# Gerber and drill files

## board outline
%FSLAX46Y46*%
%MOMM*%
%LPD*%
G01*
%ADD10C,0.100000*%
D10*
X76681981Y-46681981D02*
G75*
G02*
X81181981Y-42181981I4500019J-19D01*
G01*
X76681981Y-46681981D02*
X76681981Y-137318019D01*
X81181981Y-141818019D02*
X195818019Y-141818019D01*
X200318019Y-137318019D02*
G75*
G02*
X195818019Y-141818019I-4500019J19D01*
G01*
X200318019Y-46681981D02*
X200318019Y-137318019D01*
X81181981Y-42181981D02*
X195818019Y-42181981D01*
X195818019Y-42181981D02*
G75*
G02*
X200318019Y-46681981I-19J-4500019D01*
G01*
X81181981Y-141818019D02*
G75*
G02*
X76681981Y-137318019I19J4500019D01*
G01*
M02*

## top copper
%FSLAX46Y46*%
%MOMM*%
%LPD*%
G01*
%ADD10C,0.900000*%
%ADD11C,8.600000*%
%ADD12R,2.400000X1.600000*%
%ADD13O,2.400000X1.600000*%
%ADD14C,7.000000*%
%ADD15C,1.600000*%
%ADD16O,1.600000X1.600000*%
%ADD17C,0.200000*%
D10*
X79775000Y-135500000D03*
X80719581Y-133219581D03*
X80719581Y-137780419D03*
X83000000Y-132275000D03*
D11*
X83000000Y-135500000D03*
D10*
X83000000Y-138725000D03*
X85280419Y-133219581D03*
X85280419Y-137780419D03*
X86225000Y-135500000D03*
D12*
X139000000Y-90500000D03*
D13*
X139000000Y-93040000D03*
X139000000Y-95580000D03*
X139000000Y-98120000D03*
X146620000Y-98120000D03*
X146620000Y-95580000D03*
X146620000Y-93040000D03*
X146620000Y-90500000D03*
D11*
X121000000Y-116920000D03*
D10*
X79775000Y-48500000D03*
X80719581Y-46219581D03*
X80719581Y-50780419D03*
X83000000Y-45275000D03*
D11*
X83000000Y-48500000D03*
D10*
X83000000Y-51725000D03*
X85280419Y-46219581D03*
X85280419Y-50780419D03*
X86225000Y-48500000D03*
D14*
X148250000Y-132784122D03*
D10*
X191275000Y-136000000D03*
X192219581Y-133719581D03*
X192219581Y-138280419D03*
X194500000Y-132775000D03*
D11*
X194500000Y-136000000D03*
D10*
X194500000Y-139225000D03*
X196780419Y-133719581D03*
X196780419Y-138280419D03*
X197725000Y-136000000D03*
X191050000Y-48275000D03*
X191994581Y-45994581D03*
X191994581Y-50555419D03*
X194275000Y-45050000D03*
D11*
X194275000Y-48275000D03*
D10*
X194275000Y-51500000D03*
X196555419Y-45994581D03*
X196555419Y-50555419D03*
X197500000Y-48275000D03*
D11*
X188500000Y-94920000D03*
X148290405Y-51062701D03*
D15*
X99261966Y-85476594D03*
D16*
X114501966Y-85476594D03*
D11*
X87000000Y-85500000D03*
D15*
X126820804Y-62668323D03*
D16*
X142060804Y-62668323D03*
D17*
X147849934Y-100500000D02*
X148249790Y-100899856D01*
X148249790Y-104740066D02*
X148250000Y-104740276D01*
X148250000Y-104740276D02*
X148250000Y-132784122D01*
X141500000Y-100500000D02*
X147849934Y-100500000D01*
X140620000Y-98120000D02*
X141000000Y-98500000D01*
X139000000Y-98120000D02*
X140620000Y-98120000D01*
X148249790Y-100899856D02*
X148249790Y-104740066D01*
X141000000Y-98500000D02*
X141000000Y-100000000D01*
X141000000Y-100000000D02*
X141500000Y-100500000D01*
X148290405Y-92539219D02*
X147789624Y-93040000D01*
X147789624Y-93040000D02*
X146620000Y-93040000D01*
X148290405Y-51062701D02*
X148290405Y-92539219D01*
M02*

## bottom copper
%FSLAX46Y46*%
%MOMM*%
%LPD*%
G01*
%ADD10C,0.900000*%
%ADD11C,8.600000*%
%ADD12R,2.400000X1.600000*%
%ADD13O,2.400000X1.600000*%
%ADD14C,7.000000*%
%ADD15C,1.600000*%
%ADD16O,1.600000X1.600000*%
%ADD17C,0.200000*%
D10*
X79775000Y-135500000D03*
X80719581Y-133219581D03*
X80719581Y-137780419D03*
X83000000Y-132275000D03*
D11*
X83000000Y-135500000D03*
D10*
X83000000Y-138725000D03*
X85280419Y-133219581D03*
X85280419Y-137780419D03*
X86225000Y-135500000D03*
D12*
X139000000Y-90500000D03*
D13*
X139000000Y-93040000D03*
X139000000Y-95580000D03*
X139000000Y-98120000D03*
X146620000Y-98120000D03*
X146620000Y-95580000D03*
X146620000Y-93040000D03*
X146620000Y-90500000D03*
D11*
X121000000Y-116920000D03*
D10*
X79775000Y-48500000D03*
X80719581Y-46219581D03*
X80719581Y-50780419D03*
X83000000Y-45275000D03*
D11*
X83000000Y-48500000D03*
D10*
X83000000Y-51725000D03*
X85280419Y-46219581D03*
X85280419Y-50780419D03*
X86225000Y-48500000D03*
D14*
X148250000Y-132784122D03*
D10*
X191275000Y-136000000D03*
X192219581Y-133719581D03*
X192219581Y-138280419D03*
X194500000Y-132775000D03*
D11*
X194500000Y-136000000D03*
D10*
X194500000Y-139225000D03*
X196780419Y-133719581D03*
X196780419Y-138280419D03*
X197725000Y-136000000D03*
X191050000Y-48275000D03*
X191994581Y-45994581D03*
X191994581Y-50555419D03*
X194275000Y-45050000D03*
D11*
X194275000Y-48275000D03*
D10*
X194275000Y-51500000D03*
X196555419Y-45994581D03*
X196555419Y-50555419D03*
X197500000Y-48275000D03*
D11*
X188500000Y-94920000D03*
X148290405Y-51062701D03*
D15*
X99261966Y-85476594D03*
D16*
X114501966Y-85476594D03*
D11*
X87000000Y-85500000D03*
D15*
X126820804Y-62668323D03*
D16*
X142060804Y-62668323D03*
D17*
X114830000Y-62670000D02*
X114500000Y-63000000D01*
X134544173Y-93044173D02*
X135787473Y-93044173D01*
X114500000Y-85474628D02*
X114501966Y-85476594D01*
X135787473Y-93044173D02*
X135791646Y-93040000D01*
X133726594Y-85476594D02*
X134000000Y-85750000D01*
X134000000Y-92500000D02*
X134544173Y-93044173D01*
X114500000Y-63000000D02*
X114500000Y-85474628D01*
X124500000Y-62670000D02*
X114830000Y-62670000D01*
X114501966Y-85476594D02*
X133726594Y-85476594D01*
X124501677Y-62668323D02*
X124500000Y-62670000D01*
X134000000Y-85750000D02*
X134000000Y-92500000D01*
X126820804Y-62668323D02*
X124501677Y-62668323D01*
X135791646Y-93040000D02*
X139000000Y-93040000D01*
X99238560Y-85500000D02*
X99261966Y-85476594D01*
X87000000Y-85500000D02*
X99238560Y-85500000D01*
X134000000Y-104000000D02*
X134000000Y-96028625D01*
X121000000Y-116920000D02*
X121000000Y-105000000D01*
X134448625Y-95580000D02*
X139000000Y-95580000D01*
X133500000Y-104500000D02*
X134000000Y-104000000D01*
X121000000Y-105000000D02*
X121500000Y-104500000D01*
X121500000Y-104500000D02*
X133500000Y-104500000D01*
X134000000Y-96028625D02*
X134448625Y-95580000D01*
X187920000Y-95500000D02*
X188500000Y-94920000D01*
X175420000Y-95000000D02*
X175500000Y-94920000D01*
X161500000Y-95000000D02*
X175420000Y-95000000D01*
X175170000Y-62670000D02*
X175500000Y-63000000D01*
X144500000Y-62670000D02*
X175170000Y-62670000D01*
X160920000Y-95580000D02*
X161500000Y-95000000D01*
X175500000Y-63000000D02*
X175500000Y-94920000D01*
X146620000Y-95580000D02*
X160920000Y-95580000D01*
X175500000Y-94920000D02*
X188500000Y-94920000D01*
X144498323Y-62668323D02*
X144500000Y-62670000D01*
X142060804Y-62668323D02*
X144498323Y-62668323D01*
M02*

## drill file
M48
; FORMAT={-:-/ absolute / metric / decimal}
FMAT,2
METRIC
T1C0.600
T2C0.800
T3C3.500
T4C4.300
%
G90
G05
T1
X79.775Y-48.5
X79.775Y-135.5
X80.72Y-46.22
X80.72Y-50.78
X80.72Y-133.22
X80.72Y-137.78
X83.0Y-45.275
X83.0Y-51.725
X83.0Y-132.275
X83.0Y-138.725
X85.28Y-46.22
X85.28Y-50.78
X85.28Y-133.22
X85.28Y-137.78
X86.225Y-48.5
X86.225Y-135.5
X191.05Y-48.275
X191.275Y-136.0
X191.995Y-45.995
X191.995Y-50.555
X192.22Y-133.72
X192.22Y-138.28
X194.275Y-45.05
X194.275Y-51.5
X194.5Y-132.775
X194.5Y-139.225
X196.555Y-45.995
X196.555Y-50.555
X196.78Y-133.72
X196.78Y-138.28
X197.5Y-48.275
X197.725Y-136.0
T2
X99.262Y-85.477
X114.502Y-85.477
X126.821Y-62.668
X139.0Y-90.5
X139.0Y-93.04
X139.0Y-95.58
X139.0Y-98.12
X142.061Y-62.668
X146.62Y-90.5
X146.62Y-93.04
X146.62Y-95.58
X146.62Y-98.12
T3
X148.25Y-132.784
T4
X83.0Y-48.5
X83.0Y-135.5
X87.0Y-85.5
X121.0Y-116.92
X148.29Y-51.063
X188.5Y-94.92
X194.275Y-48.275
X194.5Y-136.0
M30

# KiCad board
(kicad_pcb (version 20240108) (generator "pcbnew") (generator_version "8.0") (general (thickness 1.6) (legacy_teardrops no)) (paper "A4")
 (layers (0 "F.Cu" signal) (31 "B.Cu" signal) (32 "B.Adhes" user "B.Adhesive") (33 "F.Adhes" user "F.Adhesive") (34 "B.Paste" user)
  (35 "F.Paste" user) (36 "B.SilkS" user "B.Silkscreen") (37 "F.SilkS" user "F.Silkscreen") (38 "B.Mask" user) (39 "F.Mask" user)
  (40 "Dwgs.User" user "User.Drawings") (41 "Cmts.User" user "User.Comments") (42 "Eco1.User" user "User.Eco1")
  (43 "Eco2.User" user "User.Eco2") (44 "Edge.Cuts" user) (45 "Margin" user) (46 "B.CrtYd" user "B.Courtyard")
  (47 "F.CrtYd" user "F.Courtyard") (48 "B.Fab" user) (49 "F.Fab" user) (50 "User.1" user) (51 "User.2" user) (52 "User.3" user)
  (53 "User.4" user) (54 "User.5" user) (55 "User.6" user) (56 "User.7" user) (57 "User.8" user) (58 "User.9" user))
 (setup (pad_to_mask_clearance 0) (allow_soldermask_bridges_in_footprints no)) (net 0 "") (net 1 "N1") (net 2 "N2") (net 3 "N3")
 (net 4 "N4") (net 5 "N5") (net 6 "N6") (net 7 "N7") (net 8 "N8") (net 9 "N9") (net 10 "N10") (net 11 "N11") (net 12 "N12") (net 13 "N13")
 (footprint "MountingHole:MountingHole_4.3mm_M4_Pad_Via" (layer "F.Cu") (at 83 135.5)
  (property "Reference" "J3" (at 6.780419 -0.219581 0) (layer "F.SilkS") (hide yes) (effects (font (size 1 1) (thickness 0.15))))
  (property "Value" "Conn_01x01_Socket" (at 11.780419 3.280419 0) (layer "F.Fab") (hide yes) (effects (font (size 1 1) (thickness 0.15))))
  (pad "1" thru_hole circle (at -3.225 0) (size 0.9 0.9) (drill 0.6) (layers "*.Cu" "*.Mask") (remove_unused_layers no) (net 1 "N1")
   (zone_connect 2))
  (pad "1" thru_hole circle (at -2.280419 -2.280419) (size 0.9 0.9) (drill 0.6) (layers "*.Cu" "*.Mask") (remove_unused_layers no)
   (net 1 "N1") (zone_connect 2))
  (pad "1" thru_hole circle (at -2.280419 2.280419) (size 0.9 0.9) (drill 0.6) (layers "*.Cu" "*.Mask") (remove_unused_layers no)
   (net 1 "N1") (zone_connect 2))
  (pad "1" thru_hole circle (at 0 -3.225) (size 0.9 0.9) (drill 0.6) (layers "*.Cu" "*.Mask") (remove_unused_layers no) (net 1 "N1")
   (zone_connect 2))
  (pad "1" thru_hole circle (at 0 0) (size 8.6 8.6) (drill 4.3) (layers "*.Cu" "*.Mask") (remove_unused_layers no) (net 1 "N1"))
  (pad "1" thru_hole circle (at 0 3.225) (size 0.9 0.9) (drill 0.6) (layers "*.Cu" "*.Mask") (remove_unused_layers no) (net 1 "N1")
   (zone_connect 2))
  (pad "1" thru_hole circle (at 2.280419 -2.280419) (size 0.9 0.9) (drill 0.6) (layers "*.Cu" "*.Mask") (remove_unused_layers no)
   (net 1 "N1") (zone_connect 2))
  (pad "1" thru_hole circle (at 2.280419 2.280419) (size 0.9 0.9) (drill 0.6) (layers "*.Cu" "*.Mask") (remove_unused_layers no)
   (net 1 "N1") (zone_connect 2))
  (pad "1" thru_hole circle (at 3.225 0) (size 0.9 0.9) (drill 0.6) (layers "*.Cu" "*.Mask") (remove_unused_layers no) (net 1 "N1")
   (zone_connect 2)))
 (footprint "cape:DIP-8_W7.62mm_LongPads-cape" (layer "F.Cu") (at 139 90.5)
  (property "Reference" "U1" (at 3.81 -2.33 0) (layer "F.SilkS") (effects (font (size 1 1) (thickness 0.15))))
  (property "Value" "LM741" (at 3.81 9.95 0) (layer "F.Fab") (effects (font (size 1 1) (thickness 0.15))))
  (pad "1" thru_hole rect (at 0 0) (size 2.4 1.6) (drill 0.8) (layers "*.Cu" "*.Mask") (remove_unused_layers no) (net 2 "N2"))
  (pad "2" thru_hole oval (at 0 2.54) (size 2.4 1.6) (drill 0.8) (layers "*.Cu" "*.Mask") (remove_unused_layers no) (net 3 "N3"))
  (pad "3" thru_hole oval (at 0 5.08) (size 2.4 1.6) (drill 0.8) (layers "*.Cu" "*.Mask") (remove_unused_layers no) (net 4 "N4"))
  (pad "4" thru_hole oval (at 0 7.62) (size 2.4 1.6) (drill 0.8) (layers "*.Cu" "*.Mask") (remove_unused_layers no) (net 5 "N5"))
  (pad "5" thru_hole oval (at 7.62 7.62) (size 2.4 1.6) (drill 0.8) (layers "*.Cu" "*.Mask") (remove_unused_layers no) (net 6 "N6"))
  (pad "6" thru_hole oval (at 7.62 5.08) (size 2.4 1.6) (drill 0.8) (layers "*.Cu" "*.Mask") (remove_unused_layers no) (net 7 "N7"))
  (pad "7" thru_hole oval (at 7.62 2.54) (size 2.4 1.6) (drill 0.8) (layers "*.Cu" "*.Mask") (remove_unused_layers no) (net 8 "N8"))
  (pad "8" thru_hole oval (at 7.62 0) (size 2.4 1.6) (drill 0.8) (layers "*.Cu" "*.Mask") (remove_unused_layers no) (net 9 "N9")))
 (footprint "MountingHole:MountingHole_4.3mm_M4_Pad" (layer "F.Cu") (at 121 116.92)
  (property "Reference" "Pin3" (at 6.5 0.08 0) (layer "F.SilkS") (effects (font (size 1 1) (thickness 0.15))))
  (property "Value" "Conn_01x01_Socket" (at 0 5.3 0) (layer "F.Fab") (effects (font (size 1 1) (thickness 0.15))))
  (pad "1" thru_hole circle (at 0 0) (size 8.6 8.6) (drill 4.3) (layers "*.Cu" "*.Mask") (remove_unused_layers no) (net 4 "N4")))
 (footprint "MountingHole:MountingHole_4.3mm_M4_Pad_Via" (layer "F.Cu") (at 83 48.5)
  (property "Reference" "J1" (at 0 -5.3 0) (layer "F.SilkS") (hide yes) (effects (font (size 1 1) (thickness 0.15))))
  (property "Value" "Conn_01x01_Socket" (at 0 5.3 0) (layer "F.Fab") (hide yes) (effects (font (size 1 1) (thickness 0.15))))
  (pad "1" thru_hole circle (at -3.225 0) (size 0.9 0.9) (drill 0.6) (layers "*.Cu" "*.Mask") (remove_unused_layers no) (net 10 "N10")
   (zone_connect 2))
  (pad "1" thru_hole circle (at -2.280419 -2.280419) (size 0.9 0.9) (drill 0.6) (layers "*.Cu" "*.Mask") (remove_unused_layers no)
   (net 10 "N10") (zone_connect 2))
  (pad "1" thru_hole circle (at -2.280419 2.280419) (size 0.9 0.9) (drill 0.6) (layers "*.Cu" "*.Mask") (remove_unused_layers no)
   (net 10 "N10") (zone_connect 2))
  (pad "1" thru_hole circle (at 0 -3.225) (size 0.9 0.9) (drill 0.6) (layers "*.Cu" "*.Mask") (remove_unused_layers no) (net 10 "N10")
   (zone_connect 2))
  (pad "1" thru_hole circle (at 0 0) (size 8.6 8.6) (drill 4.3) (layers "*.Cu" "*.Mask") (remove_unused_layers no) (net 10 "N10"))
  (pad "1" thru_hole circle (at 0 3.225) (size 0.9 0.9) (drill 0.6) (layers "*.Cu" "*.Mask") (remove_unused_layers no) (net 10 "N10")
   (zone_connect 2))
  (pad "1" thru_hole circle (at 2.280419 -2.280419) (size 0.9 0.9) (drill 0.6) (layers "*.Cu" "*.Mask") (remove_unused_layers no)
   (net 10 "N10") (zone_connect 2))
  (pad "1" thru_hole circle (at 2.280419 2.280419) (size 0.9 0.9) (drill 0.6) (layers "*.Cu" "*.Mask") (remove_unused_layers no)
   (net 10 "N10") (zone_connect 2))
  (pad "1" thru_hole circle (at 3.225 0) (size 0.9 0.9) (drill 0.6) (layers "*.Cu" "*.Mask") (remove_unused_layers no) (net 10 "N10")
   (zone_connect 2)))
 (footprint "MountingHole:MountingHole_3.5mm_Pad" (layer "F.Cu") (at 148.25 132.784122)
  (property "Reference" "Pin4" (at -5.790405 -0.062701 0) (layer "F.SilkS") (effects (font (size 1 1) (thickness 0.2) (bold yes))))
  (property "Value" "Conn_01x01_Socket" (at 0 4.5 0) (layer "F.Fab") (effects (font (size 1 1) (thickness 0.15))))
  (pad "1" thru_hole circle (at 0 0) (size 7 7) (drill 3.5) (layers "*.Cu" "*.Mask") (remove_unused_layers no) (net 5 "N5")))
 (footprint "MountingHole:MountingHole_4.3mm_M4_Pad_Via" (layer "F.Cu") (at 194.5 136)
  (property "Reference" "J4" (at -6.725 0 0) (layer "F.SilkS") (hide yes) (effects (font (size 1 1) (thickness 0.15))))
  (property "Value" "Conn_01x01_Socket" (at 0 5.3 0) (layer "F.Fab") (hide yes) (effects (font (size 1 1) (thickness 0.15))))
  (pad "1" thru_hole circle (at -3.225 0) (size 0.9 0.9) (drill 0.6) (layers "*.Cu" "*.Mask") (remove_unused_layers no) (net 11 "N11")
   (zone_connect 2))
  (pad "1" thru_hole circle (at -2.280419 -2.280419) (size 0.9 0.9) (drill 0.6) (layers "*.Cu" "*.Mask") (remove_unused_layers no)
   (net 11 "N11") (zone_connect 2))
  (pad "1" thru_hole circle (at -2.280419 2.280419) (size 0.9 0.9) (drill 0.6) (layers "*.Cu" "*.Mask") (remove_unused_layers no)
   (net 11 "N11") (zone_connect 2))
  (pad "1" thru_hole circle (at 0 -3.225) (size 0.9 0.9) (drill 0.6) (layers "*.Cu" "*.Mask") (remove_unused_layers no) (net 11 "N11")
   (zone_connect 2))
  (pad "1" thru_hole circle (at 0 0) (size 8.6 8.6) (drill 4.3) (layers "*.Cu" "*.Mask") (remove_unused_layers no) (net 11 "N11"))
  (pad "1" thru_hole circle (at 0 3.225) (size 0.9 0.9) (drill 0.6) (layers "*.Cu" "*.Mask") (remove_unused_layers no) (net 11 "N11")
   (zone_connect 2))
  (pad "1" thru_hole circle (at 2.280419 -2.280419) (size 0.9 0.9) (drill 0.6) (layers "*.Cu" "*.Mask") (remove_unused_layers no)
   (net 11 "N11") (zone_connect 2))
  (pad "1" thru_hole circle (at 2.280419 2.280419) (size 0.9 0.9) (drill 0.6) (layers "*.Cu" "*.Mask") (remove_unused_layers no)
   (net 11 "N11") (zone_connect 2))
  (pad "1" thru_hole circle (at 3.225 0) (size 0.9 0.9) (drill 0.6) (layers "*.Cu" "*.Mask") (remove_unused_layers no) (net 11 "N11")
   (zone_connect 2)))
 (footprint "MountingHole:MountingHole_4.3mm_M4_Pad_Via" (layer "F.Cu") (at 194.275 48.275)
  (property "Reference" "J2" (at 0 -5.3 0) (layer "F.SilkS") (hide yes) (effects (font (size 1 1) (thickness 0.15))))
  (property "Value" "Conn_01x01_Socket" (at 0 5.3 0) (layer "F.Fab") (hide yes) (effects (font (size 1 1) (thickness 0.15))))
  (pad "1" thru_hole circle (at -3.225 0) (size 0.9 0.9) (drill 0.6) (layers "*.Cu" "*.Mask") (remove_unused_layers no) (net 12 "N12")
   (zone_connect 2))
  (pad "1" thru_hole circle (at -2.280419 -2.280419) (size 0.9 0.9) (drill 0.6) (layers "*.Cu" "*.Mask") (remove_unused_layers no)
   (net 12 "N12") (zone_connect 2))
  (pad "1" thru_hole circle (at -2.280419 2.280419) (size 0.9 0.9) (drill 0.6) (layers "*.Cu" "*.Mask") (remove_unused_layers no)
   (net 12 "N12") (zone_connect 2))
  (pad "1" thru_hole circle (at 0 -3.225) (size 0.9 0.9) (drill 0.6) (layers "*.Cu" "*.Mask") (remove_unused_layers no) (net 12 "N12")
   (zone_connect 2))
  (pad "1" thru_hole circle (at 0 0) (size 8.6 8.6) (drill 4.3) (layers "*.Cu" "*.Mask") (remove_unused_layers no) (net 12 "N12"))
  (pad "1" thru_hole circle (at 0 3.225) (size 0.9 0.9) (drill 0.6) (layers "*.Cu" "*.Mask") (remove_unused_layers no) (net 12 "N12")
   (zone_connect 2))
  (pad "1" thru_hole circle (at 2.280419 -2.280419) (size 0.9 0.9) (drill 0.6) (layers "*.Cu" "*.Mask") (remove_unused_layers no)
   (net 12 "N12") (zone_connect 2))
  (pad "1" thru_hole circle (at 2.280419 2.280419) (size 0.9 0.9) (drill 0.6) (layers "*.Cu" "*.Mask") (remove_unused_layers no)
   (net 12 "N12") (zone_connect 2))
  (pad "1" thru_hole circle (at 3.225 0) (size 0.9 0.9) (drill 0.6) (layers "*.Cu" "*.Mask") (remove_unused_layers no) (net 12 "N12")
   (zone_connect 2)))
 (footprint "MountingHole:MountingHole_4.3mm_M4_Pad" (layer "F.Cu") (at 188.5 94.92)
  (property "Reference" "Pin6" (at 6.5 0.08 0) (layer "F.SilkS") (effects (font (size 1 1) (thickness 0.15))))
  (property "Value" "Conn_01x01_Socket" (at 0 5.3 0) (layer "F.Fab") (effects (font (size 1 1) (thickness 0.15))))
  (pad "1" thru_hole circle (at 0 0) (size 8.6 8.6) (drill 4.3) (layers "*.Cu" "*.Mask") (remove_unused_layers no) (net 7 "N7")))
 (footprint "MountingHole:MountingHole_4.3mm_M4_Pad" (layer "F.Cu") (at 148.290405 51.062701)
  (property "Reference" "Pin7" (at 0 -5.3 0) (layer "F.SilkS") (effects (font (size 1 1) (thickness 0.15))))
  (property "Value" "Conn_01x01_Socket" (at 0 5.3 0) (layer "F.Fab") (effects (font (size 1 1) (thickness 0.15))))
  (pad "1" thru_hole circle (at 0 0) (size 8.6 8.6) (drill 4.3) (layers "*.Cu" "*.Mask") (remove_unused_layers no) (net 8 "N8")))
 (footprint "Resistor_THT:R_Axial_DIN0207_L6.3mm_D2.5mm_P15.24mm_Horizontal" (layer "F.Cu") (at 99.261966 85.476594)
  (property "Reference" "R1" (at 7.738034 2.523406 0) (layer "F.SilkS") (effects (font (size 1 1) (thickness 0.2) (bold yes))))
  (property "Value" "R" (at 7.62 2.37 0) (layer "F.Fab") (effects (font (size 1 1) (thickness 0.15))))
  (pad "1" thru_hole circle (at 0 0) (size 1.6 1.6) (drill 0.8) (layers "*.Cu" "*.Mask") (remove_unused_layers no) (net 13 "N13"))
  (pad "2" thru_hole oval (at 15.24 0) (size 1.6 1.6) (drill 0.8) (layers "*.Cu" "*.Mask") (remove_unused_layers no) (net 3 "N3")))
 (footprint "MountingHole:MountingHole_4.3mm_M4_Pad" (layer "F.Cu") (at 87 85.5)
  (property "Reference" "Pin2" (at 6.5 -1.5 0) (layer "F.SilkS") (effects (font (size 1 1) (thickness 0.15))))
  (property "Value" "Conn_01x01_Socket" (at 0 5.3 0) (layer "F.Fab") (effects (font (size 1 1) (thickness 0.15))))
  (pad "1" thru_hole circle (at 0 0) (size 8.6 8.6) (drill 4.3) (layers "*.Cu" "*.Mask") (remove_unused_layers no) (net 13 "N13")))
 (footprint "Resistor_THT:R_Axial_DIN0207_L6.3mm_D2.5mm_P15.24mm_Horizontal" (layer "F.Cu") (at 126.820804 62.668323)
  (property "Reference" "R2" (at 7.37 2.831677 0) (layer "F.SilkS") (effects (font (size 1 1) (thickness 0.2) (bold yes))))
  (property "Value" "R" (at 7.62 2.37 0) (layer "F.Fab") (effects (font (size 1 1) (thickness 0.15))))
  (pad "1" thru_hole circle (at 0 0) (size 1.6 1.6) (drill 0.8) (layers "*.Cu" "*.Mask") (remove_unused_layers no) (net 3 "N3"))
  (pad "2" thru_hole oval (at 15.24 0) (size 1.6 1.6) (drill 0.8) (layers "*.Cu" "*.Mask") (remove_unused_layers no) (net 7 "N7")))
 (gr_arc (start 76.681981 46.681981) (mid 78 43.5) (end 81.181981 42.181981) (stroke (width 0.1) (type default)) (layer "Edge.Cuts"))
 (gr_line (start 76.681981 46.681981) (end 76.681981 137.318019) (stroke (width 0.1) (type default)) (layer "Edge.Cuts"))
 (gr_line (start 81.181981 141.818019) (end 195.818019 141.818019) (stroke (width 0.1) (type default)) (layer "Edge.Cuts"))
 (gr_arc (start 200.318019 137.318019) (mid 199 140.5) (end 195.818019 141.818019) (stroke (width 0.1) (type default)) (layer "Edge.Cuts"))
 (gr_line (start 200.318019 46.681981) (end 200.318019 137.318019) (stroke (width 0.1) (type default)) (layer "Edge.Cuts"))
 (gr_line (start 81.181981 42.181981) (end 195.818019 42.181981) (stroke (width 0.1) (type default)) (layer "Edge.Cuts"))
 (gr_arc (start 195.818019 42.181981) (mid 199 43.5) (end 200.318019 46.681981) (stroke (width 0.1) (type default)) (layer "Edge.Cuts"))
 (gr_arc (start 81.181981 141.818019) (mid 78 140.5) (end 76.681981 137.318019) (stroke (width 0.1) (type default)) (layer "Edge.Cuts"))
 (segment (start 114.83 62.67) (end 114.5 63) (width 0.2) (layer "B.Cu") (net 3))
 (segment (start 134.544173 93.044173) (end 135.787473 93.044173) (width 0.2) (layer "B.Cu") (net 3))
 (segment (start 114.5 85.474628) (end 114.501966 85.476594) (width 0.2) (layer "B.Cu") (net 3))
 (segment (start 135.787473 93.044173) (end 135.791646 93.04) (width 0.2) (layer "B.Cu") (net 3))
 (segment (start 133.726594 85.476594) (end 134 85.75) (width 0.2) (layer "B.Cu") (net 3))
 (segment (start 134 92.5) (end 134.544173 93.044173) (width 0.2) (layer "B.Cu") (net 3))
 (segment (start 114.5 63) (end 114.5 85.474628) (width 0.2) (layer "B.Cu") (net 3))
 (segment (start 124.5 62.67) (end 114.83 62.67) (width 0.2) (layer "B.Cu") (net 3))
 (segment (start 114.501966 85.476594) (end 133.726594 85.476594) (width 0.2) (layer "B.Cu") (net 3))
 (segment (start 124.501677 62.668323) (end 124.5 62.67) (width 0.2) (layer "B.Cu") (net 3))
 (segment (start 134 85.75) (end 134 92.5) (width 0.2) (layer "B.Cu") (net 3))
 (segment (start 126.820804 62.668323) (end 124.501677 62.668323) (width 0.2) (layer "B.Cu") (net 3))
 (segment (start 135.791646 93.04) (end 139 93.04) (width 0.2) (layer "B.Cu") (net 3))
 (segment (start 99.23856 85.5) (end 99.261966 85.476594) (width 0.2) (layer "B.Cu") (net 13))
 (segment (start 87 85.5) (end 99.23856 85.5) (width 0.2) (layer "B.Cu") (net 13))
 (segment (start 134 104) (end 134 96.028625) (width 0.2) (layer "B.Cu") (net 4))
 (segment (start 121 116.92) (end 121 105) (width 0.2) (layer "B.Cu") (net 4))
 (segment (start 134.448625 95.58) (end 139 95.58) (width 0.2) (layer "B.Cu") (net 4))
 (segment (start 133.5 104.5) (end 134 104) (width 0.2) (layer "B.Cu") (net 4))
 (segment (start 121 105) (end 121.5 104.5) (width 0.2) (layer "B.Cu") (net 4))
 (segment (start 121.5 104.5) (end 133.5 104.5) (width 0.2) (layer "B.Cu") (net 4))
 (segment (start 134 96.028625) (end 134.448625 95.58) (width 0.2) (layer "B.Cu") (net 4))
 (segment (start 147.849934 100.5) (end 148.24979 100.899856) (width 0.2) (layer "F.Cu") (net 5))
 (segment (start 148.24979 104.740066) (end 148.25 104.740276) (width 0.2) (layer "F.Cu") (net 5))
 (segment (start 148.25 104.740276) (end 148.25 132.784122) (width 0.2) (layer "F.Cu") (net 5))
 (segment (start 141.5 100.5) (end 147.849934 100.5) (width 0.2) (layer "F.Cu") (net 5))
 (segment (start 140.62 98.12) (end 141 98.5) (width 0.2) (layer "F.Cu") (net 5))
 (segment (start 139 98.12) (end 140.62 98.12) (width 0.2) (layer "F.Cu") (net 5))
 (segment (start 148.24979 100.899856) (end 148.24979 104.740066) (width 0.2) (layer "F.Cu") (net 5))
 (segment (start 141 98.5) (end 141 100) (width 0.2) (layer "F.Cu") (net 5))
 (segment (start 141 100) (end 141.5 100.5) (width 0.2) (layer "F.Cu") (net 5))
 (segment (start 187.92 95.5) (end 188.5 94.92) (width 0.2) (layer "B.Cu") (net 7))
 (segment (start 175.42 95) (end 175.5 94.92) (width 0.2) (layer "B.Cu") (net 7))
 (segment (start 161.5 95) (end 175.42 95) (width 0.2) (layer "B.Cu") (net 7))
 (segment (start 175.17 62.67) (end 175.5 63) (width 0.2) (layer "B.Cu") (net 7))
 (segment (start 144.5 62.67) (end 175.17 62.67) (width 0.2) (layer "B.Cu") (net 7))
 (segment (start 160.92 95.58) (end 161.5 95) (width 0.2) (layer "B.Cu") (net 7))
 (segment (start 175.5 63) (end 175.5 94.92) (width 0.2) (layer "B.Cu") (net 7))
 (segment (start 146.62 95.58) (end 160.92 95.58) (width 0.2) (layer "B.Cu") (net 7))
 (segment (start 175.5 94.92) (end 188.5 94.92) (width 0.2) (layer "B.Cu") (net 7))
 (segment (start 144.498323 62.668323) (end 144.5 62.67) (width 0.2) (layer "B.Cu") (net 7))
 (segment (start 142.060804 62.668323) (end 144.498323 62.668323) (width 0.2) (layer "B.Cu") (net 7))
 (segment (start 148.290405 92.539219) (end 147.789624 93.04) (width 0.2) (layer "F.Cu") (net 8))
 (segment (start 147.789624 93.04) (end 146.62 93.04) (width 0.2) (layer "F.Cu") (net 8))
 (segment (start 148.290405 51.062701) (end 148.290405 92.539219) (width 0.2) (layer "F.Cu") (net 8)))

